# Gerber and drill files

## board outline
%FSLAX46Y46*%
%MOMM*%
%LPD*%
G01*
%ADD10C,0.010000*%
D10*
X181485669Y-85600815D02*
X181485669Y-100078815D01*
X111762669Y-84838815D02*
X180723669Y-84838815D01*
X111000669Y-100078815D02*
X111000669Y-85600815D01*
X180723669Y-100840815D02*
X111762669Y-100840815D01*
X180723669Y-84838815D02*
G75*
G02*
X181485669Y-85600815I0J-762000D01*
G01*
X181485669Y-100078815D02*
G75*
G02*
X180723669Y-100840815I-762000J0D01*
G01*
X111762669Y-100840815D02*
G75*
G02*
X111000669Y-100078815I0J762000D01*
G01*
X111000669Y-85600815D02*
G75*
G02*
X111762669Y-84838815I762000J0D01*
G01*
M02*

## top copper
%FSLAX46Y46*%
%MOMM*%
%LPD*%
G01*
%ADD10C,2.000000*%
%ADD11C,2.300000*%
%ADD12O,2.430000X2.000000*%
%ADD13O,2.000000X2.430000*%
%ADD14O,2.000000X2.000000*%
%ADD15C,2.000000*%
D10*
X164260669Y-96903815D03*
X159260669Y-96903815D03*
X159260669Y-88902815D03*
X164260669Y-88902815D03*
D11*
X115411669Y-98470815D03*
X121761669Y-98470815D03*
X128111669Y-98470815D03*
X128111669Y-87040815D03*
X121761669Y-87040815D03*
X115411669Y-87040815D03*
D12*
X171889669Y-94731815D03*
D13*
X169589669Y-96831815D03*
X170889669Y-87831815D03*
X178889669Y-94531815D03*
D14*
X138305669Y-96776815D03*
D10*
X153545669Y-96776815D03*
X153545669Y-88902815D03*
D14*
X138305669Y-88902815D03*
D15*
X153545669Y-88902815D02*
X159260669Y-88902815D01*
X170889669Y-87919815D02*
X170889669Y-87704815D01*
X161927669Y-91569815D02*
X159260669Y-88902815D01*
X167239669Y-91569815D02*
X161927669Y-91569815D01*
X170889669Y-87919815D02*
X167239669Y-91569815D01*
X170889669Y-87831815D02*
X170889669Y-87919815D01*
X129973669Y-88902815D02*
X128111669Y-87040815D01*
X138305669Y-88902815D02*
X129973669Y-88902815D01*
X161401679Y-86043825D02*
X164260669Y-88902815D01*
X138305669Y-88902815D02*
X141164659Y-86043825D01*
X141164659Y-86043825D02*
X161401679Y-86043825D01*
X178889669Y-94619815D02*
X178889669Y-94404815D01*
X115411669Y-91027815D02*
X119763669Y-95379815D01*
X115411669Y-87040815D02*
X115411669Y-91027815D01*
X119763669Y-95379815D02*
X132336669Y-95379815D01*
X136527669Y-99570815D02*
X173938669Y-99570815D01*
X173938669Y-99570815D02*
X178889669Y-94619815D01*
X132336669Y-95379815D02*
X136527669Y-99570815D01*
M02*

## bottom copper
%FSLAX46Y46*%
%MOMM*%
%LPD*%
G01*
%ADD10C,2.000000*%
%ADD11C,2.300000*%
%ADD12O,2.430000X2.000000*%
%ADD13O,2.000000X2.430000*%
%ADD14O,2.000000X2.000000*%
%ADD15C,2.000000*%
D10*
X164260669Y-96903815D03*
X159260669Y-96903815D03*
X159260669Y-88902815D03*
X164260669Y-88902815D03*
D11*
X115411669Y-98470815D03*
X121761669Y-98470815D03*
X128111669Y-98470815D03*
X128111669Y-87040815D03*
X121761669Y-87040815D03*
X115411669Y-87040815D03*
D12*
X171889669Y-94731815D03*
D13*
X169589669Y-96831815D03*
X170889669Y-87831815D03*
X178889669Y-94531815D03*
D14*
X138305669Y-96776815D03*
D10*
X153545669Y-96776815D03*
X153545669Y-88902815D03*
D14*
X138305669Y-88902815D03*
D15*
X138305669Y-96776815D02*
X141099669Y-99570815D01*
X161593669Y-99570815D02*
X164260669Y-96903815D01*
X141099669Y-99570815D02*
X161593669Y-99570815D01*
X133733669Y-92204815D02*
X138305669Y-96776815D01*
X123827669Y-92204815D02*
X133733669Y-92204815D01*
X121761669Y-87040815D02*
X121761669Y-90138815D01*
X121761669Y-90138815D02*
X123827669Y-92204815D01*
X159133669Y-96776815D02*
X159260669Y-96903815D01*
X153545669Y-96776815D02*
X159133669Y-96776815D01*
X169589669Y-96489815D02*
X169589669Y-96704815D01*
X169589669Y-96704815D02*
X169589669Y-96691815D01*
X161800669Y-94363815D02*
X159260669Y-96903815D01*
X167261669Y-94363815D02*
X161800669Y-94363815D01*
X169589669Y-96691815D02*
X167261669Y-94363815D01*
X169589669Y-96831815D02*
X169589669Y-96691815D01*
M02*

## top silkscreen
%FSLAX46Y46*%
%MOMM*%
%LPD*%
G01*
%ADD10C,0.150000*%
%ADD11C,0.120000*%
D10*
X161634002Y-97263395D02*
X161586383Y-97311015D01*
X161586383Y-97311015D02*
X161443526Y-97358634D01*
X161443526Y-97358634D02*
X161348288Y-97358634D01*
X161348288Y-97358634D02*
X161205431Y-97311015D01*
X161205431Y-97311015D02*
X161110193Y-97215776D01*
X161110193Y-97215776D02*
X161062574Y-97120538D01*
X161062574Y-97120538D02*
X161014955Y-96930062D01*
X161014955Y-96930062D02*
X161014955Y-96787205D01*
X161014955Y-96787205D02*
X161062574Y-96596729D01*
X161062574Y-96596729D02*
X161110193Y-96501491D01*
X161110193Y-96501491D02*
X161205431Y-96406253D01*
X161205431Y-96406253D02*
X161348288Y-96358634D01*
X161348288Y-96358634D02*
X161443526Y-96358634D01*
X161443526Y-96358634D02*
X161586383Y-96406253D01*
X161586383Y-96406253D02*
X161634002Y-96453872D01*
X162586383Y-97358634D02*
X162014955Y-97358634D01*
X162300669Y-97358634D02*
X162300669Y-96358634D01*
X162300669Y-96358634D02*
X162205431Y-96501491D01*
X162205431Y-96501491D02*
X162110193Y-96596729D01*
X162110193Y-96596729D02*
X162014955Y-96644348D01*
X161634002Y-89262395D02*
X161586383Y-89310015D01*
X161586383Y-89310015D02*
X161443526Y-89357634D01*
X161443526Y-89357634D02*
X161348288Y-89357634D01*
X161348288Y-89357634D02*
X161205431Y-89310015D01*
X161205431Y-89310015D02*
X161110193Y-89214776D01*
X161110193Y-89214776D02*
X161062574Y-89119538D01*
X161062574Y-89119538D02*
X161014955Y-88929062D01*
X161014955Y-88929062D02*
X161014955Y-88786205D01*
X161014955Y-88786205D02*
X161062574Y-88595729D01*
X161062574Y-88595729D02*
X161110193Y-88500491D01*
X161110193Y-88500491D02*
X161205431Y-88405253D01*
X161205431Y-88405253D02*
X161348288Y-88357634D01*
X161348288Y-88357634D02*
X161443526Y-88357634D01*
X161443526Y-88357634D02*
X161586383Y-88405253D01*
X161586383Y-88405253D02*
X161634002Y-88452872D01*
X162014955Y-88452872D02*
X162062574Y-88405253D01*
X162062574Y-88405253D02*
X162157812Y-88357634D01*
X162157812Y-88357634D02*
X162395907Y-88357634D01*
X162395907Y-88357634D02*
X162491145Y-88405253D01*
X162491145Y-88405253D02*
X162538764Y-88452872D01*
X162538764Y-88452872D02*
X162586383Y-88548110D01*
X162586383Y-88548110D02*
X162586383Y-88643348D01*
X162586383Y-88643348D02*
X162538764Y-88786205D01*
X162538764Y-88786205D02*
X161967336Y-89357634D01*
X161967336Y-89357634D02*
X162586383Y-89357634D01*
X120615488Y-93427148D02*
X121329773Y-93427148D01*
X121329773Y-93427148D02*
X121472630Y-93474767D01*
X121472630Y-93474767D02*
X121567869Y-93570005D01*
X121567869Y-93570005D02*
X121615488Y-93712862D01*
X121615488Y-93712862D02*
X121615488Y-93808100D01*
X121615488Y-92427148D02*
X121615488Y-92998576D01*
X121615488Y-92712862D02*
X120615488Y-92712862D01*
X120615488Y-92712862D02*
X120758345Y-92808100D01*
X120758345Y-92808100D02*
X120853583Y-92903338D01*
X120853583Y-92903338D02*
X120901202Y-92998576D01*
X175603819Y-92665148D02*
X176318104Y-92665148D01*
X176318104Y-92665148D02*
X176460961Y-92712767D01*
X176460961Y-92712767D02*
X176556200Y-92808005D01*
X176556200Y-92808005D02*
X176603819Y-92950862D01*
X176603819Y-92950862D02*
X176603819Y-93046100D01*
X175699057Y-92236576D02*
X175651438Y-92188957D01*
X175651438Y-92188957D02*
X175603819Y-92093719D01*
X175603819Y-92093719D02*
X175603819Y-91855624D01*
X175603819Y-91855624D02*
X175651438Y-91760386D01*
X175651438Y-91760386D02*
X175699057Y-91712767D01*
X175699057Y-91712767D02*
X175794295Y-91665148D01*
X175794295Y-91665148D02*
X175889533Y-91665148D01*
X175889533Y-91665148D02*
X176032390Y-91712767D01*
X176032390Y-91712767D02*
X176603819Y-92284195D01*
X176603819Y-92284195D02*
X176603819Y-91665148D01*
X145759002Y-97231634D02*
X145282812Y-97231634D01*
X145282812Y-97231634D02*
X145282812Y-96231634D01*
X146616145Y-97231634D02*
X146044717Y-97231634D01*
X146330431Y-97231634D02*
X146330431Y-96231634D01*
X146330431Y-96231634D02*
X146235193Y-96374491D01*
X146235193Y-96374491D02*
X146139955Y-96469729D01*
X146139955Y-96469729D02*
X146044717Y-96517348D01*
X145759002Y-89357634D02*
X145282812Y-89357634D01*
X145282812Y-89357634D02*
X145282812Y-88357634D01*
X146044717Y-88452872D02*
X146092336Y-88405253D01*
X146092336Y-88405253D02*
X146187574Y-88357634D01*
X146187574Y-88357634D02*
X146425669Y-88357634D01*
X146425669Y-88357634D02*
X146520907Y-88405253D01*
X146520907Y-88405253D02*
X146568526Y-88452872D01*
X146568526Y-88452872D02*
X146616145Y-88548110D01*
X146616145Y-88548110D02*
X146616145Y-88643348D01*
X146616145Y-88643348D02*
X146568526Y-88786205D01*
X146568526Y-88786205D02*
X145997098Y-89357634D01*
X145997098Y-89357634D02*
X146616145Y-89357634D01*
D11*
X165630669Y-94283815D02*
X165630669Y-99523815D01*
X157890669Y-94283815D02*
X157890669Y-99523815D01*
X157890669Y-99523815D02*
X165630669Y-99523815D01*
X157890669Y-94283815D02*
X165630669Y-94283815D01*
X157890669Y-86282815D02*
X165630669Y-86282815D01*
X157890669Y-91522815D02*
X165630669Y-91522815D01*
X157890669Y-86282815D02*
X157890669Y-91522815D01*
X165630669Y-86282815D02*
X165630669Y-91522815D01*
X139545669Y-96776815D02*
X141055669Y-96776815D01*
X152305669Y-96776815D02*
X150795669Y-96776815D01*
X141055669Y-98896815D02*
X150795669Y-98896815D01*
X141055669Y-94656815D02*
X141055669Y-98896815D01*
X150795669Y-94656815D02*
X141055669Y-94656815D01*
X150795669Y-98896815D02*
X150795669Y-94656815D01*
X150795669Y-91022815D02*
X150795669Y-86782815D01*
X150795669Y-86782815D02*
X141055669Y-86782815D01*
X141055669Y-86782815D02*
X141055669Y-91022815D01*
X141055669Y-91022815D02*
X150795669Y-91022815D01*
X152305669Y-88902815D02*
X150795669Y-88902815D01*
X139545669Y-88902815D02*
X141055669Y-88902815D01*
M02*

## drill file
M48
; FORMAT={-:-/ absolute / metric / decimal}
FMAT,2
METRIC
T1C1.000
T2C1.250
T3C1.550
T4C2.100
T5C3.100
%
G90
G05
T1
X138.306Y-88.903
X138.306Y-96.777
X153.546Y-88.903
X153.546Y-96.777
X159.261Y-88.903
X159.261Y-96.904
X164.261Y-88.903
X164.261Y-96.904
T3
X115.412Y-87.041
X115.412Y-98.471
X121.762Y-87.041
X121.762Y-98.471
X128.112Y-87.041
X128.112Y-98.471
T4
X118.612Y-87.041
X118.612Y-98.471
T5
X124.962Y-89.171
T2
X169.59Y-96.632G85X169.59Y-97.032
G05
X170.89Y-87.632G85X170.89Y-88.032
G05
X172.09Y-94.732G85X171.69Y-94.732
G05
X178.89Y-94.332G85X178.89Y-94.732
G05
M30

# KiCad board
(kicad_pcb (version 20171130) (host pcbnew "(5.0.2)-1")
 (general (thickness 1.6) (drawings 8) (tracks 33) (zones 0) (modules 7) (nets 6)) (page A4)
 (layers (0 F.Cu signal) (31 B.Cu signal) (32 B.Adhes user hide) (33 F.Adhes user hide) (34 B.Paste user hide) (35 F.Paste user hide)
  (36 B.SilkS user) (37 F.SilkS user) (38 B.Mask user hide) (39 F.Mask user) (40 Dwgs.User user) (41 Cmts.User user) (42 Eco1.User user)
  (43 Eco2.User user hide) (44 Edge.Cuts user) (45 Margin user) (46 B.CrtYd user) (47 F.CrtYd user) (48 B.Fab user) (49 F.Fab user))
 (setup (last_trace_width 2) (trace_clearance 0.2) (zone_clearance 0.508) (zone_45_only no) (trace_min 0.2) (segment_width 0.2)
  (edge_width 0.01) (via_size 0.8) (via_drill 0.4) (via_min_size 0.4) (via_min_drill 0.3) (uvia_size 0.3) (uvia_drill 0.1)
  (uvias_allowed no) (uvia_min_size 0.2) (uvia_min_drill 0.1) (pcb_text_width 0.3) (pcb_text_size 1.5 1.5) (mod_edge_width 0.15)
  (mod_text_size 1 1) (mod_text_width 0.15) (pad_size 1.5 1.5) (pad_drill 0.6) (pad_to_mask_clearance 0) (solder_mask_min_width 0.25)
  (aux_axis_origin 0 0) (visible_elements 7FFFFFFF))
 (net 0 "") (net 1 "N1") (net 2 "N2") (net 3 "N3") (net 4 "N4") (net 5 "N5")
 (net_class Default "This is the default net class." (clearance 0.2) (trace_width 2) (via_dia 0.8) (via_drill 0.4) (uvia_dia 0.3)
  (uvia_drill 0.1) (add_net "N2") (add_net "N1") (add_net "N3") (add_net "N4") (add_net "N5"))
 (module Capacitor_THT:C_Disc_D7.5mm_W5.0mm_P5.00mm (layer F.Cu) (at 159.260669 96.903815)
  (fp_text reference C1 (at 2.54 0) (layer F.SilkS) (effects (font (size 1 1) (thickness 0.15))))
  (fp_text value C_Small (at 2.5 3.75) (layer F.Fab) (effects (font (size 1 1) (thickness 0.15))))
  (fp_line (start 6.37 -2.62) (end 6.37 2.62) (layer F.SilkS) (width 0.12))
  (fp_line (start -1.37 -2.62) (end -1.37 2.62) (layer F.SilkS) (width 0.12))
  (fp_line (start -1.37 2.62) (end 6.37 2.62) (layer F.SilkS) (width 0.12))
  (fp_line (start -1.37 -2.62) (end 6.37 -2.62) (layer F.SilkS) (width 0.12))
  (pad 2 thru_hole circle (at 5 0) (size 2 2) (drill 1) (layers *.Cu *.Mask) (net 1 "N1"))
  (pad 1 thru_hole circle (at 0 0) (size 2 2) (drill 1) (layers *.Cu *.Mask) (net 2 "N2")))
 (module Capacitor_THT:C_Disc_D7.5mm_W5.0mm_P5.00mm (layer F.Cu) (at 159.260669 88.902815)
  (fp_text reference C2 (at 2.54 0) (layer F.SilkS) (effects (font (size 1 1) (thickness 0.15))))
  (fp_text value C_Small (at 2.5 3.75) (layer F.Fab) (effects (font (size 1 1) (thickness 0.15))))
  (fp_line (start -1.37 -2.62) (end 6.37 -2.62) (layer F.SilkS) (width 0.12))
  (fp_line (start -1.37 2.62) (end 6.37 2.62) (layer F.SilkS) (width 0.12))
  (fp_line (start -1.37 -2.62) (end -1.37 2.62) (layer F.SilkS) (width 0.12))
  (fp_line (start 6.37 -2.62) (end 6.37 2.62) (layer F.SilkS) (width 0.12))
  (pad 1 thru_hole circle (at 0 0) (size 2 2) (drill 1) (layers *.Cu *.Mask) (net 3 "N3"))
  (pad 2 thru_hole circle (at 5 0) (size 2 2) (drill 1) (layers *.Cu *.Mask) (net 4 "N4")))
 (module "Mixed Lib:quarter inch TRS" (layer B.Cu) (at 111.161669 94.270815 270)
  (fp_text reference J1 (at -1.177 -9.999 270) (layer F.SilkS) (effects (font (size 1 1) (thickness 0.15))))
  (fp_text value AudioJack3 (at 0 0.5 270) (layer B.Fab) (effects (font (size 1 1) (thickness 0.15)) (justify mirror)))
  (pad SN thru_hole circle (at 4.2 -4.25 270) (size 2.3 2.3) (drill 1.55) (layers *.Cu *.Mask))
  (pad RN thru_hole circle (at 4.2 -10.6 270) (size 2.3 2.3) (drill 1.55) (layers *.Cu *.Mask))
  (pad TN thru_hole circle (at 4.2 -16.95 270) (size 2.3 2.3) (drill 1.55) (layers *.Cu *.Mask))
  (pad T thru_hole circle (at -7.23 -16.95 270) (size 2.3 2.3) (drill 1.55) (layers *.Cu *.Mask) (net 4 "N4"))
  (pad R thru_hole circle (at -7.23 -10.6 270) (size 2.3 2.3) (drill 1.55) (layers *.Cu *.Mask) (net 1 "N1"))
  (pad S thru_hole circle (at -7.23 -4.25 270) (size 2.3 2.3) (drill 1.55) (layers *.Cu *.Mask) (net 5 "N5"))
  (pad "" np_thru_hole circle (at -7.23 -7.45 270) (size 2.1 2.1) (drill 2.1) (layers *.Cu *.Mask))
  (pad "" np_thru_hole circle (at 4.2 -7.45 270) (size 2.1 2.1) (drill 2.1) (layers *.Cu *.Mask))
  (pad "" np_thru_hole circle (at -5.1 -13.8 270) (size 3.1 3.1) (drill 3.1) (layers *.Cu *.Mask)))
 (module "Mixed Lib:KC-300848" (layer F.Cu) (at 175.389669 92.331815 270)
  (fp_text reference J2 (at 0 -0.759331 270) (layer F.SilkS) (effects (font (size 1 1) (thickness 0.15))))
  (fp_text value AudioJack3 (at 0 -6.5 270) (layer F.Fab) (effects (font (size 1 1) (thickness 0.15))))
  (pad B thru_hole oval (at 2.4 3.5 180) (size 2.43 2) (drill oval 1.65 1.25) (layers *.Cu *.Mask))
  (pad R thru_hole oval (at 4.5 5.8 270) (size 2.43 2) (drill oval 1.65 1.25) (layers *.Cu *.Mask) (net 2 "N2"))
  (pad T thru_hole oval (at -4.5 4.5 270) (size 2.43 2) (drill oval 1.65 1.25) (layers *.Cu *.Mask) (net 3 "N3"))
  (pad S thru_hole oval (at 2.2 -3.5 270) (size 2.43 2) (drill oval 1.65 1.25) (layers *.Cu *.Mask) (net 5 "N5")))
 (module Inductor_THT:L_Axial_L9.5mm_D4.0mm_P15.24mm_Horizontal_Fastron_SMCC (layer F.Cu) (at 153.545669 96.776815 180)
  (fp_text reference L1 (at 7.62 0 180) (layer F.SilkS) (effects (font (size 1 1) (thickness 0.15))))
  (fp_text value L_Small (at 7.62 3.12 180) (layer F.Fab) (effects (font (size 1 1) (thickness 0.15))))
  (fp_line (start 14 0) (end 12.49 0) (layer F.SilkS) (width 0.12))
  (fp_line (start 1.24 0) (end 2.75 0) (layer F.SilkS) (width 0.12))
  (fp_line (start 12.49 -2.12) (end 2.75 -2.12) (layer F.SilkS) (width 0.12))
  (fp_line (start 12.49 2.12) (end 12.49 -2.12) (layer F.SilkS) (width 0.12))
  (fp_line (start 2.75 2.12) (end 12.49 2.12) (layer F.SilkS) (width 0.12))
  (fp_line (start 2.75 -2.12) (end 2.75 2.12) (layer F.SilkS) (width 0.12))
  (pad 2 thru_hole oval (at 15.24 0 180) (size 2 2) (drill 1) (layers *.Cu *.Mask) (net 1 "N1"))
  (pad 1 thru_hole circle (at 0 0 180) (size 2 2) (drill 1) (layers *.Cu *.Mask) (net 2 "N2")))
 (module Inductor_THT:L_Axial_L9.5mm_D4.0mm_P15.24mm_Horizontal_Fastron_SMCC (layer F.Cu) (at 153.545669 88.902815 180)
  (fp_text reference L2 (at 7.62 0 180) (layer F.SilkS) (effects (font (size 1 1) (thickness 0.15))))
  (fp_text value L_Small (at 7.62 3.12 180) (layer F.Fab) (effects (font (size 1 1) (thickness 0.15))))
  (fp_line (start 2.75 -2.12) (end 2.75 2.12) (layer F.SilkS) (width 0.12))
  (fp_line (start 2.75 2.12) (end 12.49 2.12) (layer F.SilkS) (width 0.12))
  (fp_line (start 12.49 2.12) (end 12.49 -2.12) (layer F.SilkS) (width 0.12))
  (fp_line (start 12.49 -2.12) (end 2.75 -2.12) (layer F.SilkS) (width 0.12))
  (fp_line (start 1.24 0) (end 2.75 0) (layer F.SilkS) (width 0.12))
  (fp_line (start 14 0) (end 12.49 0) (layer F.SilkS) (width 0.12))
  (pad 1 thru_hole circle (at 0 0 180) (size 2 2) (drill 1) (layers *.Cu *.Mask) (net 3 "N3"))
  (pad 2 thru_hole oval (at 15.24 0 180) (size 2 2) (drill 1) (layers *.Cu *.Mask) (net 4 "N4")))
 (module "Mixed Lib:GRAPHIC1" (layer B.Cu) (at 146.179669 92.839815 180)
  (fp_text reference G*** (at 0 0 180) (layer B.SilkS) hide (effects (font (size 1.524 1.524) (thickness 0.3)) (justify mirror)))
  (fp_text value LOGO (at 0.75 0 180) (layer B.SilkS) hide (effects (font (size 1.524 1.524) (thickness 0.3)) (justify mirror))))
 (gr_line (start 181.485669 85.600815) (end 181.485669 100.078815) (layer Edge.Cuts) (width 0.01))
 (gr_line (start 111.762669 84.838815) (end 180.723669 84.838815) (layer Edge.Cuts) (width 0.01))
 (gr_line (start 111.000669 100.078815) (end 111.000669 85.600815) (layer Edge.Cuts) (width 0.01))
 (gr_line (start 180.723669 100.840815) (end 111.762669 100.840815) (layer Edge.Cuts) (width 0.01))
 (gr_arc (start 180.723669 85.600815) (end 180.723669 84.838815) (angle 90) (layer Edge.Cuts) (width 0.01))
 (gr_arc (start 180.723669 100.078815) (end 181.485669 100.078815) (angle 90) (layer Edge.Cuts) (width 0.01))
 (gr_arc (start 111.762669 100.078815) (end 111.000669 100.078815) (angle -90) (layer Edge.Cuts) (width 0.01))
 (gr_arc (start 111.762669 85.600815) (end 111.762669 84.838815) (angle -90) (layer Edge.Cuts) (width 0.01))
 (segment (start 138.305669 96.776815) (end 141.099669 99.570815) (width 2) (layer B.Cu) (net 1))
 (segment (start 161.593669 99.570815) (end 164.260669 96.903815) (width 2) (layer B.Cu) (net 1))
 (segment (start 141.099669 99.570815) (end 161.593669 99.570815) (width 2) (layer B.Cu) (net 1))
 (segment (start 133.733669 92.204815) (end 138.305669 96.776815) (width 2) (layer B.Cu) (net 1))
 (segment (start 123.827669 92.204815) (end 133.733669 92.204815) (width 2) (layer B.Cu) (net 1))
 (segment (start 121.761669 87.040815) (end 121.761669 90.138815) (width 2) (layer B.Cu) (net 1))
 (segment (start 121.761669 90.138815) (end 123.827669 92.204815) (width 2) (layer B.Cu) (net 1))
 (segment (start 159.133669 96.776815) (end 159.260669 96.903815) (width 2) (layer B.Cu) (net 2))
 (segment (start 153.545669 96.776815) (end 159.133669 96.776815) (width 2) (layer B.Cu) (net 2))
 (segment (start 169.589669 96.489815) (end 169.589669 96.704815) (width 2) (layer B.Cu) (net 2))
 (segment (start 169.589669 96.704815) (end 169.589669 96.691815) (width 2) (layer B.Cu) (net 2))
 (segment (start 161.800669 94.363815) (end 159.260669 96.903815) (width 2) (layer B.Cu) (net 2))
 (segment (start 167.261669 94.363815) (end 161.800669 94.363815) (width 2) (layer B.Cu) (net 2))
 (segment (start 169.589669 96.691815) (end 167.261669 94.363815) (width 2) (layer B.Cu) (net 2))
 (segment (start 169.589669 96.831815) (end 169.589669 96.691815) (width 2) (layer B.Cu) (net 2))
 (segment (start 153.545669 88.902815) (end 159.260669 88.902815) (width 2) (layer F.Cu) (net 3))
 (segment (start 170.889669 87.919815) (end 170.889669 87.704815) (width 2) (layer F.Cu) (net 3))
 (segment (start 161.927669 91.569815) (end 159.260669 88.902815) (width 2) (layer F.Cu) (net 3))
 (segment (start 167.239669 91.569815) (end 161.927669 91.569815) (width 2) (layer F.Cu) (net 3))
 (segment (start 170.889669 87.919815) (end 167.239669 91.569815) (width 2) (layer F.Cu) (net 3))
 (segment (start 170.889669 87.831815) (end 170.889669 87.919815) (width 2) (layer F.Cu) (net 3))
 (segment (start 129.973669 88.902815) (end 128.111669 87.040815) (width 2) (layer F.Cu) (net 4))
 (segment (start 138.305669 88.902815) (end 129.973669 88.902815) (width 2) (layer F.Cu) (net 4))
 (segment (start 161.401679 86.043825) (end 164.260669 88.902815) (width 2) (layer F.Cu) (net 4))
 (segment (start 138.305669 88.902815) (end 141.164659 86.043825) (width 2) (layer F.Cu) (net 4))
 (segment (start 141.164659 86.043825) (end 161.401679 86.043825) (width 2) (layer F.Cu) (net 4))
 (segment (start 178.889669 94.619815) (end 178.889669 94.404815) (width 2) (layer F.Cu) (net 5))
 (segment (start 115.411669 91.027815) (end 119.763669 95.379815) (width 2) (layer F.Cu) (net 5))
 (segment (start 115.411669 87.040815) (end 115.411669 91.027815) (width 2) (layer F.Cu) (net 5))
 (segment (start 119.763669 95.379815) (end 132.336669 95.379815) (width 2) (layer F.Cu) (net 5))
 (segment (start 136.527669 99.570815) (end 173.938669 99.570815) (width 2) (layer F.Cu) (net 5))
 (segment (start 173.938669 99.570815) (end 178.889669 94.619815) (width 2) (layer F.Cu) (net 5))
 (segment (start 132.336669 95.379815) (end 136.527669 99.570815) (width 2) (layer F.Cu) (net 5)))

